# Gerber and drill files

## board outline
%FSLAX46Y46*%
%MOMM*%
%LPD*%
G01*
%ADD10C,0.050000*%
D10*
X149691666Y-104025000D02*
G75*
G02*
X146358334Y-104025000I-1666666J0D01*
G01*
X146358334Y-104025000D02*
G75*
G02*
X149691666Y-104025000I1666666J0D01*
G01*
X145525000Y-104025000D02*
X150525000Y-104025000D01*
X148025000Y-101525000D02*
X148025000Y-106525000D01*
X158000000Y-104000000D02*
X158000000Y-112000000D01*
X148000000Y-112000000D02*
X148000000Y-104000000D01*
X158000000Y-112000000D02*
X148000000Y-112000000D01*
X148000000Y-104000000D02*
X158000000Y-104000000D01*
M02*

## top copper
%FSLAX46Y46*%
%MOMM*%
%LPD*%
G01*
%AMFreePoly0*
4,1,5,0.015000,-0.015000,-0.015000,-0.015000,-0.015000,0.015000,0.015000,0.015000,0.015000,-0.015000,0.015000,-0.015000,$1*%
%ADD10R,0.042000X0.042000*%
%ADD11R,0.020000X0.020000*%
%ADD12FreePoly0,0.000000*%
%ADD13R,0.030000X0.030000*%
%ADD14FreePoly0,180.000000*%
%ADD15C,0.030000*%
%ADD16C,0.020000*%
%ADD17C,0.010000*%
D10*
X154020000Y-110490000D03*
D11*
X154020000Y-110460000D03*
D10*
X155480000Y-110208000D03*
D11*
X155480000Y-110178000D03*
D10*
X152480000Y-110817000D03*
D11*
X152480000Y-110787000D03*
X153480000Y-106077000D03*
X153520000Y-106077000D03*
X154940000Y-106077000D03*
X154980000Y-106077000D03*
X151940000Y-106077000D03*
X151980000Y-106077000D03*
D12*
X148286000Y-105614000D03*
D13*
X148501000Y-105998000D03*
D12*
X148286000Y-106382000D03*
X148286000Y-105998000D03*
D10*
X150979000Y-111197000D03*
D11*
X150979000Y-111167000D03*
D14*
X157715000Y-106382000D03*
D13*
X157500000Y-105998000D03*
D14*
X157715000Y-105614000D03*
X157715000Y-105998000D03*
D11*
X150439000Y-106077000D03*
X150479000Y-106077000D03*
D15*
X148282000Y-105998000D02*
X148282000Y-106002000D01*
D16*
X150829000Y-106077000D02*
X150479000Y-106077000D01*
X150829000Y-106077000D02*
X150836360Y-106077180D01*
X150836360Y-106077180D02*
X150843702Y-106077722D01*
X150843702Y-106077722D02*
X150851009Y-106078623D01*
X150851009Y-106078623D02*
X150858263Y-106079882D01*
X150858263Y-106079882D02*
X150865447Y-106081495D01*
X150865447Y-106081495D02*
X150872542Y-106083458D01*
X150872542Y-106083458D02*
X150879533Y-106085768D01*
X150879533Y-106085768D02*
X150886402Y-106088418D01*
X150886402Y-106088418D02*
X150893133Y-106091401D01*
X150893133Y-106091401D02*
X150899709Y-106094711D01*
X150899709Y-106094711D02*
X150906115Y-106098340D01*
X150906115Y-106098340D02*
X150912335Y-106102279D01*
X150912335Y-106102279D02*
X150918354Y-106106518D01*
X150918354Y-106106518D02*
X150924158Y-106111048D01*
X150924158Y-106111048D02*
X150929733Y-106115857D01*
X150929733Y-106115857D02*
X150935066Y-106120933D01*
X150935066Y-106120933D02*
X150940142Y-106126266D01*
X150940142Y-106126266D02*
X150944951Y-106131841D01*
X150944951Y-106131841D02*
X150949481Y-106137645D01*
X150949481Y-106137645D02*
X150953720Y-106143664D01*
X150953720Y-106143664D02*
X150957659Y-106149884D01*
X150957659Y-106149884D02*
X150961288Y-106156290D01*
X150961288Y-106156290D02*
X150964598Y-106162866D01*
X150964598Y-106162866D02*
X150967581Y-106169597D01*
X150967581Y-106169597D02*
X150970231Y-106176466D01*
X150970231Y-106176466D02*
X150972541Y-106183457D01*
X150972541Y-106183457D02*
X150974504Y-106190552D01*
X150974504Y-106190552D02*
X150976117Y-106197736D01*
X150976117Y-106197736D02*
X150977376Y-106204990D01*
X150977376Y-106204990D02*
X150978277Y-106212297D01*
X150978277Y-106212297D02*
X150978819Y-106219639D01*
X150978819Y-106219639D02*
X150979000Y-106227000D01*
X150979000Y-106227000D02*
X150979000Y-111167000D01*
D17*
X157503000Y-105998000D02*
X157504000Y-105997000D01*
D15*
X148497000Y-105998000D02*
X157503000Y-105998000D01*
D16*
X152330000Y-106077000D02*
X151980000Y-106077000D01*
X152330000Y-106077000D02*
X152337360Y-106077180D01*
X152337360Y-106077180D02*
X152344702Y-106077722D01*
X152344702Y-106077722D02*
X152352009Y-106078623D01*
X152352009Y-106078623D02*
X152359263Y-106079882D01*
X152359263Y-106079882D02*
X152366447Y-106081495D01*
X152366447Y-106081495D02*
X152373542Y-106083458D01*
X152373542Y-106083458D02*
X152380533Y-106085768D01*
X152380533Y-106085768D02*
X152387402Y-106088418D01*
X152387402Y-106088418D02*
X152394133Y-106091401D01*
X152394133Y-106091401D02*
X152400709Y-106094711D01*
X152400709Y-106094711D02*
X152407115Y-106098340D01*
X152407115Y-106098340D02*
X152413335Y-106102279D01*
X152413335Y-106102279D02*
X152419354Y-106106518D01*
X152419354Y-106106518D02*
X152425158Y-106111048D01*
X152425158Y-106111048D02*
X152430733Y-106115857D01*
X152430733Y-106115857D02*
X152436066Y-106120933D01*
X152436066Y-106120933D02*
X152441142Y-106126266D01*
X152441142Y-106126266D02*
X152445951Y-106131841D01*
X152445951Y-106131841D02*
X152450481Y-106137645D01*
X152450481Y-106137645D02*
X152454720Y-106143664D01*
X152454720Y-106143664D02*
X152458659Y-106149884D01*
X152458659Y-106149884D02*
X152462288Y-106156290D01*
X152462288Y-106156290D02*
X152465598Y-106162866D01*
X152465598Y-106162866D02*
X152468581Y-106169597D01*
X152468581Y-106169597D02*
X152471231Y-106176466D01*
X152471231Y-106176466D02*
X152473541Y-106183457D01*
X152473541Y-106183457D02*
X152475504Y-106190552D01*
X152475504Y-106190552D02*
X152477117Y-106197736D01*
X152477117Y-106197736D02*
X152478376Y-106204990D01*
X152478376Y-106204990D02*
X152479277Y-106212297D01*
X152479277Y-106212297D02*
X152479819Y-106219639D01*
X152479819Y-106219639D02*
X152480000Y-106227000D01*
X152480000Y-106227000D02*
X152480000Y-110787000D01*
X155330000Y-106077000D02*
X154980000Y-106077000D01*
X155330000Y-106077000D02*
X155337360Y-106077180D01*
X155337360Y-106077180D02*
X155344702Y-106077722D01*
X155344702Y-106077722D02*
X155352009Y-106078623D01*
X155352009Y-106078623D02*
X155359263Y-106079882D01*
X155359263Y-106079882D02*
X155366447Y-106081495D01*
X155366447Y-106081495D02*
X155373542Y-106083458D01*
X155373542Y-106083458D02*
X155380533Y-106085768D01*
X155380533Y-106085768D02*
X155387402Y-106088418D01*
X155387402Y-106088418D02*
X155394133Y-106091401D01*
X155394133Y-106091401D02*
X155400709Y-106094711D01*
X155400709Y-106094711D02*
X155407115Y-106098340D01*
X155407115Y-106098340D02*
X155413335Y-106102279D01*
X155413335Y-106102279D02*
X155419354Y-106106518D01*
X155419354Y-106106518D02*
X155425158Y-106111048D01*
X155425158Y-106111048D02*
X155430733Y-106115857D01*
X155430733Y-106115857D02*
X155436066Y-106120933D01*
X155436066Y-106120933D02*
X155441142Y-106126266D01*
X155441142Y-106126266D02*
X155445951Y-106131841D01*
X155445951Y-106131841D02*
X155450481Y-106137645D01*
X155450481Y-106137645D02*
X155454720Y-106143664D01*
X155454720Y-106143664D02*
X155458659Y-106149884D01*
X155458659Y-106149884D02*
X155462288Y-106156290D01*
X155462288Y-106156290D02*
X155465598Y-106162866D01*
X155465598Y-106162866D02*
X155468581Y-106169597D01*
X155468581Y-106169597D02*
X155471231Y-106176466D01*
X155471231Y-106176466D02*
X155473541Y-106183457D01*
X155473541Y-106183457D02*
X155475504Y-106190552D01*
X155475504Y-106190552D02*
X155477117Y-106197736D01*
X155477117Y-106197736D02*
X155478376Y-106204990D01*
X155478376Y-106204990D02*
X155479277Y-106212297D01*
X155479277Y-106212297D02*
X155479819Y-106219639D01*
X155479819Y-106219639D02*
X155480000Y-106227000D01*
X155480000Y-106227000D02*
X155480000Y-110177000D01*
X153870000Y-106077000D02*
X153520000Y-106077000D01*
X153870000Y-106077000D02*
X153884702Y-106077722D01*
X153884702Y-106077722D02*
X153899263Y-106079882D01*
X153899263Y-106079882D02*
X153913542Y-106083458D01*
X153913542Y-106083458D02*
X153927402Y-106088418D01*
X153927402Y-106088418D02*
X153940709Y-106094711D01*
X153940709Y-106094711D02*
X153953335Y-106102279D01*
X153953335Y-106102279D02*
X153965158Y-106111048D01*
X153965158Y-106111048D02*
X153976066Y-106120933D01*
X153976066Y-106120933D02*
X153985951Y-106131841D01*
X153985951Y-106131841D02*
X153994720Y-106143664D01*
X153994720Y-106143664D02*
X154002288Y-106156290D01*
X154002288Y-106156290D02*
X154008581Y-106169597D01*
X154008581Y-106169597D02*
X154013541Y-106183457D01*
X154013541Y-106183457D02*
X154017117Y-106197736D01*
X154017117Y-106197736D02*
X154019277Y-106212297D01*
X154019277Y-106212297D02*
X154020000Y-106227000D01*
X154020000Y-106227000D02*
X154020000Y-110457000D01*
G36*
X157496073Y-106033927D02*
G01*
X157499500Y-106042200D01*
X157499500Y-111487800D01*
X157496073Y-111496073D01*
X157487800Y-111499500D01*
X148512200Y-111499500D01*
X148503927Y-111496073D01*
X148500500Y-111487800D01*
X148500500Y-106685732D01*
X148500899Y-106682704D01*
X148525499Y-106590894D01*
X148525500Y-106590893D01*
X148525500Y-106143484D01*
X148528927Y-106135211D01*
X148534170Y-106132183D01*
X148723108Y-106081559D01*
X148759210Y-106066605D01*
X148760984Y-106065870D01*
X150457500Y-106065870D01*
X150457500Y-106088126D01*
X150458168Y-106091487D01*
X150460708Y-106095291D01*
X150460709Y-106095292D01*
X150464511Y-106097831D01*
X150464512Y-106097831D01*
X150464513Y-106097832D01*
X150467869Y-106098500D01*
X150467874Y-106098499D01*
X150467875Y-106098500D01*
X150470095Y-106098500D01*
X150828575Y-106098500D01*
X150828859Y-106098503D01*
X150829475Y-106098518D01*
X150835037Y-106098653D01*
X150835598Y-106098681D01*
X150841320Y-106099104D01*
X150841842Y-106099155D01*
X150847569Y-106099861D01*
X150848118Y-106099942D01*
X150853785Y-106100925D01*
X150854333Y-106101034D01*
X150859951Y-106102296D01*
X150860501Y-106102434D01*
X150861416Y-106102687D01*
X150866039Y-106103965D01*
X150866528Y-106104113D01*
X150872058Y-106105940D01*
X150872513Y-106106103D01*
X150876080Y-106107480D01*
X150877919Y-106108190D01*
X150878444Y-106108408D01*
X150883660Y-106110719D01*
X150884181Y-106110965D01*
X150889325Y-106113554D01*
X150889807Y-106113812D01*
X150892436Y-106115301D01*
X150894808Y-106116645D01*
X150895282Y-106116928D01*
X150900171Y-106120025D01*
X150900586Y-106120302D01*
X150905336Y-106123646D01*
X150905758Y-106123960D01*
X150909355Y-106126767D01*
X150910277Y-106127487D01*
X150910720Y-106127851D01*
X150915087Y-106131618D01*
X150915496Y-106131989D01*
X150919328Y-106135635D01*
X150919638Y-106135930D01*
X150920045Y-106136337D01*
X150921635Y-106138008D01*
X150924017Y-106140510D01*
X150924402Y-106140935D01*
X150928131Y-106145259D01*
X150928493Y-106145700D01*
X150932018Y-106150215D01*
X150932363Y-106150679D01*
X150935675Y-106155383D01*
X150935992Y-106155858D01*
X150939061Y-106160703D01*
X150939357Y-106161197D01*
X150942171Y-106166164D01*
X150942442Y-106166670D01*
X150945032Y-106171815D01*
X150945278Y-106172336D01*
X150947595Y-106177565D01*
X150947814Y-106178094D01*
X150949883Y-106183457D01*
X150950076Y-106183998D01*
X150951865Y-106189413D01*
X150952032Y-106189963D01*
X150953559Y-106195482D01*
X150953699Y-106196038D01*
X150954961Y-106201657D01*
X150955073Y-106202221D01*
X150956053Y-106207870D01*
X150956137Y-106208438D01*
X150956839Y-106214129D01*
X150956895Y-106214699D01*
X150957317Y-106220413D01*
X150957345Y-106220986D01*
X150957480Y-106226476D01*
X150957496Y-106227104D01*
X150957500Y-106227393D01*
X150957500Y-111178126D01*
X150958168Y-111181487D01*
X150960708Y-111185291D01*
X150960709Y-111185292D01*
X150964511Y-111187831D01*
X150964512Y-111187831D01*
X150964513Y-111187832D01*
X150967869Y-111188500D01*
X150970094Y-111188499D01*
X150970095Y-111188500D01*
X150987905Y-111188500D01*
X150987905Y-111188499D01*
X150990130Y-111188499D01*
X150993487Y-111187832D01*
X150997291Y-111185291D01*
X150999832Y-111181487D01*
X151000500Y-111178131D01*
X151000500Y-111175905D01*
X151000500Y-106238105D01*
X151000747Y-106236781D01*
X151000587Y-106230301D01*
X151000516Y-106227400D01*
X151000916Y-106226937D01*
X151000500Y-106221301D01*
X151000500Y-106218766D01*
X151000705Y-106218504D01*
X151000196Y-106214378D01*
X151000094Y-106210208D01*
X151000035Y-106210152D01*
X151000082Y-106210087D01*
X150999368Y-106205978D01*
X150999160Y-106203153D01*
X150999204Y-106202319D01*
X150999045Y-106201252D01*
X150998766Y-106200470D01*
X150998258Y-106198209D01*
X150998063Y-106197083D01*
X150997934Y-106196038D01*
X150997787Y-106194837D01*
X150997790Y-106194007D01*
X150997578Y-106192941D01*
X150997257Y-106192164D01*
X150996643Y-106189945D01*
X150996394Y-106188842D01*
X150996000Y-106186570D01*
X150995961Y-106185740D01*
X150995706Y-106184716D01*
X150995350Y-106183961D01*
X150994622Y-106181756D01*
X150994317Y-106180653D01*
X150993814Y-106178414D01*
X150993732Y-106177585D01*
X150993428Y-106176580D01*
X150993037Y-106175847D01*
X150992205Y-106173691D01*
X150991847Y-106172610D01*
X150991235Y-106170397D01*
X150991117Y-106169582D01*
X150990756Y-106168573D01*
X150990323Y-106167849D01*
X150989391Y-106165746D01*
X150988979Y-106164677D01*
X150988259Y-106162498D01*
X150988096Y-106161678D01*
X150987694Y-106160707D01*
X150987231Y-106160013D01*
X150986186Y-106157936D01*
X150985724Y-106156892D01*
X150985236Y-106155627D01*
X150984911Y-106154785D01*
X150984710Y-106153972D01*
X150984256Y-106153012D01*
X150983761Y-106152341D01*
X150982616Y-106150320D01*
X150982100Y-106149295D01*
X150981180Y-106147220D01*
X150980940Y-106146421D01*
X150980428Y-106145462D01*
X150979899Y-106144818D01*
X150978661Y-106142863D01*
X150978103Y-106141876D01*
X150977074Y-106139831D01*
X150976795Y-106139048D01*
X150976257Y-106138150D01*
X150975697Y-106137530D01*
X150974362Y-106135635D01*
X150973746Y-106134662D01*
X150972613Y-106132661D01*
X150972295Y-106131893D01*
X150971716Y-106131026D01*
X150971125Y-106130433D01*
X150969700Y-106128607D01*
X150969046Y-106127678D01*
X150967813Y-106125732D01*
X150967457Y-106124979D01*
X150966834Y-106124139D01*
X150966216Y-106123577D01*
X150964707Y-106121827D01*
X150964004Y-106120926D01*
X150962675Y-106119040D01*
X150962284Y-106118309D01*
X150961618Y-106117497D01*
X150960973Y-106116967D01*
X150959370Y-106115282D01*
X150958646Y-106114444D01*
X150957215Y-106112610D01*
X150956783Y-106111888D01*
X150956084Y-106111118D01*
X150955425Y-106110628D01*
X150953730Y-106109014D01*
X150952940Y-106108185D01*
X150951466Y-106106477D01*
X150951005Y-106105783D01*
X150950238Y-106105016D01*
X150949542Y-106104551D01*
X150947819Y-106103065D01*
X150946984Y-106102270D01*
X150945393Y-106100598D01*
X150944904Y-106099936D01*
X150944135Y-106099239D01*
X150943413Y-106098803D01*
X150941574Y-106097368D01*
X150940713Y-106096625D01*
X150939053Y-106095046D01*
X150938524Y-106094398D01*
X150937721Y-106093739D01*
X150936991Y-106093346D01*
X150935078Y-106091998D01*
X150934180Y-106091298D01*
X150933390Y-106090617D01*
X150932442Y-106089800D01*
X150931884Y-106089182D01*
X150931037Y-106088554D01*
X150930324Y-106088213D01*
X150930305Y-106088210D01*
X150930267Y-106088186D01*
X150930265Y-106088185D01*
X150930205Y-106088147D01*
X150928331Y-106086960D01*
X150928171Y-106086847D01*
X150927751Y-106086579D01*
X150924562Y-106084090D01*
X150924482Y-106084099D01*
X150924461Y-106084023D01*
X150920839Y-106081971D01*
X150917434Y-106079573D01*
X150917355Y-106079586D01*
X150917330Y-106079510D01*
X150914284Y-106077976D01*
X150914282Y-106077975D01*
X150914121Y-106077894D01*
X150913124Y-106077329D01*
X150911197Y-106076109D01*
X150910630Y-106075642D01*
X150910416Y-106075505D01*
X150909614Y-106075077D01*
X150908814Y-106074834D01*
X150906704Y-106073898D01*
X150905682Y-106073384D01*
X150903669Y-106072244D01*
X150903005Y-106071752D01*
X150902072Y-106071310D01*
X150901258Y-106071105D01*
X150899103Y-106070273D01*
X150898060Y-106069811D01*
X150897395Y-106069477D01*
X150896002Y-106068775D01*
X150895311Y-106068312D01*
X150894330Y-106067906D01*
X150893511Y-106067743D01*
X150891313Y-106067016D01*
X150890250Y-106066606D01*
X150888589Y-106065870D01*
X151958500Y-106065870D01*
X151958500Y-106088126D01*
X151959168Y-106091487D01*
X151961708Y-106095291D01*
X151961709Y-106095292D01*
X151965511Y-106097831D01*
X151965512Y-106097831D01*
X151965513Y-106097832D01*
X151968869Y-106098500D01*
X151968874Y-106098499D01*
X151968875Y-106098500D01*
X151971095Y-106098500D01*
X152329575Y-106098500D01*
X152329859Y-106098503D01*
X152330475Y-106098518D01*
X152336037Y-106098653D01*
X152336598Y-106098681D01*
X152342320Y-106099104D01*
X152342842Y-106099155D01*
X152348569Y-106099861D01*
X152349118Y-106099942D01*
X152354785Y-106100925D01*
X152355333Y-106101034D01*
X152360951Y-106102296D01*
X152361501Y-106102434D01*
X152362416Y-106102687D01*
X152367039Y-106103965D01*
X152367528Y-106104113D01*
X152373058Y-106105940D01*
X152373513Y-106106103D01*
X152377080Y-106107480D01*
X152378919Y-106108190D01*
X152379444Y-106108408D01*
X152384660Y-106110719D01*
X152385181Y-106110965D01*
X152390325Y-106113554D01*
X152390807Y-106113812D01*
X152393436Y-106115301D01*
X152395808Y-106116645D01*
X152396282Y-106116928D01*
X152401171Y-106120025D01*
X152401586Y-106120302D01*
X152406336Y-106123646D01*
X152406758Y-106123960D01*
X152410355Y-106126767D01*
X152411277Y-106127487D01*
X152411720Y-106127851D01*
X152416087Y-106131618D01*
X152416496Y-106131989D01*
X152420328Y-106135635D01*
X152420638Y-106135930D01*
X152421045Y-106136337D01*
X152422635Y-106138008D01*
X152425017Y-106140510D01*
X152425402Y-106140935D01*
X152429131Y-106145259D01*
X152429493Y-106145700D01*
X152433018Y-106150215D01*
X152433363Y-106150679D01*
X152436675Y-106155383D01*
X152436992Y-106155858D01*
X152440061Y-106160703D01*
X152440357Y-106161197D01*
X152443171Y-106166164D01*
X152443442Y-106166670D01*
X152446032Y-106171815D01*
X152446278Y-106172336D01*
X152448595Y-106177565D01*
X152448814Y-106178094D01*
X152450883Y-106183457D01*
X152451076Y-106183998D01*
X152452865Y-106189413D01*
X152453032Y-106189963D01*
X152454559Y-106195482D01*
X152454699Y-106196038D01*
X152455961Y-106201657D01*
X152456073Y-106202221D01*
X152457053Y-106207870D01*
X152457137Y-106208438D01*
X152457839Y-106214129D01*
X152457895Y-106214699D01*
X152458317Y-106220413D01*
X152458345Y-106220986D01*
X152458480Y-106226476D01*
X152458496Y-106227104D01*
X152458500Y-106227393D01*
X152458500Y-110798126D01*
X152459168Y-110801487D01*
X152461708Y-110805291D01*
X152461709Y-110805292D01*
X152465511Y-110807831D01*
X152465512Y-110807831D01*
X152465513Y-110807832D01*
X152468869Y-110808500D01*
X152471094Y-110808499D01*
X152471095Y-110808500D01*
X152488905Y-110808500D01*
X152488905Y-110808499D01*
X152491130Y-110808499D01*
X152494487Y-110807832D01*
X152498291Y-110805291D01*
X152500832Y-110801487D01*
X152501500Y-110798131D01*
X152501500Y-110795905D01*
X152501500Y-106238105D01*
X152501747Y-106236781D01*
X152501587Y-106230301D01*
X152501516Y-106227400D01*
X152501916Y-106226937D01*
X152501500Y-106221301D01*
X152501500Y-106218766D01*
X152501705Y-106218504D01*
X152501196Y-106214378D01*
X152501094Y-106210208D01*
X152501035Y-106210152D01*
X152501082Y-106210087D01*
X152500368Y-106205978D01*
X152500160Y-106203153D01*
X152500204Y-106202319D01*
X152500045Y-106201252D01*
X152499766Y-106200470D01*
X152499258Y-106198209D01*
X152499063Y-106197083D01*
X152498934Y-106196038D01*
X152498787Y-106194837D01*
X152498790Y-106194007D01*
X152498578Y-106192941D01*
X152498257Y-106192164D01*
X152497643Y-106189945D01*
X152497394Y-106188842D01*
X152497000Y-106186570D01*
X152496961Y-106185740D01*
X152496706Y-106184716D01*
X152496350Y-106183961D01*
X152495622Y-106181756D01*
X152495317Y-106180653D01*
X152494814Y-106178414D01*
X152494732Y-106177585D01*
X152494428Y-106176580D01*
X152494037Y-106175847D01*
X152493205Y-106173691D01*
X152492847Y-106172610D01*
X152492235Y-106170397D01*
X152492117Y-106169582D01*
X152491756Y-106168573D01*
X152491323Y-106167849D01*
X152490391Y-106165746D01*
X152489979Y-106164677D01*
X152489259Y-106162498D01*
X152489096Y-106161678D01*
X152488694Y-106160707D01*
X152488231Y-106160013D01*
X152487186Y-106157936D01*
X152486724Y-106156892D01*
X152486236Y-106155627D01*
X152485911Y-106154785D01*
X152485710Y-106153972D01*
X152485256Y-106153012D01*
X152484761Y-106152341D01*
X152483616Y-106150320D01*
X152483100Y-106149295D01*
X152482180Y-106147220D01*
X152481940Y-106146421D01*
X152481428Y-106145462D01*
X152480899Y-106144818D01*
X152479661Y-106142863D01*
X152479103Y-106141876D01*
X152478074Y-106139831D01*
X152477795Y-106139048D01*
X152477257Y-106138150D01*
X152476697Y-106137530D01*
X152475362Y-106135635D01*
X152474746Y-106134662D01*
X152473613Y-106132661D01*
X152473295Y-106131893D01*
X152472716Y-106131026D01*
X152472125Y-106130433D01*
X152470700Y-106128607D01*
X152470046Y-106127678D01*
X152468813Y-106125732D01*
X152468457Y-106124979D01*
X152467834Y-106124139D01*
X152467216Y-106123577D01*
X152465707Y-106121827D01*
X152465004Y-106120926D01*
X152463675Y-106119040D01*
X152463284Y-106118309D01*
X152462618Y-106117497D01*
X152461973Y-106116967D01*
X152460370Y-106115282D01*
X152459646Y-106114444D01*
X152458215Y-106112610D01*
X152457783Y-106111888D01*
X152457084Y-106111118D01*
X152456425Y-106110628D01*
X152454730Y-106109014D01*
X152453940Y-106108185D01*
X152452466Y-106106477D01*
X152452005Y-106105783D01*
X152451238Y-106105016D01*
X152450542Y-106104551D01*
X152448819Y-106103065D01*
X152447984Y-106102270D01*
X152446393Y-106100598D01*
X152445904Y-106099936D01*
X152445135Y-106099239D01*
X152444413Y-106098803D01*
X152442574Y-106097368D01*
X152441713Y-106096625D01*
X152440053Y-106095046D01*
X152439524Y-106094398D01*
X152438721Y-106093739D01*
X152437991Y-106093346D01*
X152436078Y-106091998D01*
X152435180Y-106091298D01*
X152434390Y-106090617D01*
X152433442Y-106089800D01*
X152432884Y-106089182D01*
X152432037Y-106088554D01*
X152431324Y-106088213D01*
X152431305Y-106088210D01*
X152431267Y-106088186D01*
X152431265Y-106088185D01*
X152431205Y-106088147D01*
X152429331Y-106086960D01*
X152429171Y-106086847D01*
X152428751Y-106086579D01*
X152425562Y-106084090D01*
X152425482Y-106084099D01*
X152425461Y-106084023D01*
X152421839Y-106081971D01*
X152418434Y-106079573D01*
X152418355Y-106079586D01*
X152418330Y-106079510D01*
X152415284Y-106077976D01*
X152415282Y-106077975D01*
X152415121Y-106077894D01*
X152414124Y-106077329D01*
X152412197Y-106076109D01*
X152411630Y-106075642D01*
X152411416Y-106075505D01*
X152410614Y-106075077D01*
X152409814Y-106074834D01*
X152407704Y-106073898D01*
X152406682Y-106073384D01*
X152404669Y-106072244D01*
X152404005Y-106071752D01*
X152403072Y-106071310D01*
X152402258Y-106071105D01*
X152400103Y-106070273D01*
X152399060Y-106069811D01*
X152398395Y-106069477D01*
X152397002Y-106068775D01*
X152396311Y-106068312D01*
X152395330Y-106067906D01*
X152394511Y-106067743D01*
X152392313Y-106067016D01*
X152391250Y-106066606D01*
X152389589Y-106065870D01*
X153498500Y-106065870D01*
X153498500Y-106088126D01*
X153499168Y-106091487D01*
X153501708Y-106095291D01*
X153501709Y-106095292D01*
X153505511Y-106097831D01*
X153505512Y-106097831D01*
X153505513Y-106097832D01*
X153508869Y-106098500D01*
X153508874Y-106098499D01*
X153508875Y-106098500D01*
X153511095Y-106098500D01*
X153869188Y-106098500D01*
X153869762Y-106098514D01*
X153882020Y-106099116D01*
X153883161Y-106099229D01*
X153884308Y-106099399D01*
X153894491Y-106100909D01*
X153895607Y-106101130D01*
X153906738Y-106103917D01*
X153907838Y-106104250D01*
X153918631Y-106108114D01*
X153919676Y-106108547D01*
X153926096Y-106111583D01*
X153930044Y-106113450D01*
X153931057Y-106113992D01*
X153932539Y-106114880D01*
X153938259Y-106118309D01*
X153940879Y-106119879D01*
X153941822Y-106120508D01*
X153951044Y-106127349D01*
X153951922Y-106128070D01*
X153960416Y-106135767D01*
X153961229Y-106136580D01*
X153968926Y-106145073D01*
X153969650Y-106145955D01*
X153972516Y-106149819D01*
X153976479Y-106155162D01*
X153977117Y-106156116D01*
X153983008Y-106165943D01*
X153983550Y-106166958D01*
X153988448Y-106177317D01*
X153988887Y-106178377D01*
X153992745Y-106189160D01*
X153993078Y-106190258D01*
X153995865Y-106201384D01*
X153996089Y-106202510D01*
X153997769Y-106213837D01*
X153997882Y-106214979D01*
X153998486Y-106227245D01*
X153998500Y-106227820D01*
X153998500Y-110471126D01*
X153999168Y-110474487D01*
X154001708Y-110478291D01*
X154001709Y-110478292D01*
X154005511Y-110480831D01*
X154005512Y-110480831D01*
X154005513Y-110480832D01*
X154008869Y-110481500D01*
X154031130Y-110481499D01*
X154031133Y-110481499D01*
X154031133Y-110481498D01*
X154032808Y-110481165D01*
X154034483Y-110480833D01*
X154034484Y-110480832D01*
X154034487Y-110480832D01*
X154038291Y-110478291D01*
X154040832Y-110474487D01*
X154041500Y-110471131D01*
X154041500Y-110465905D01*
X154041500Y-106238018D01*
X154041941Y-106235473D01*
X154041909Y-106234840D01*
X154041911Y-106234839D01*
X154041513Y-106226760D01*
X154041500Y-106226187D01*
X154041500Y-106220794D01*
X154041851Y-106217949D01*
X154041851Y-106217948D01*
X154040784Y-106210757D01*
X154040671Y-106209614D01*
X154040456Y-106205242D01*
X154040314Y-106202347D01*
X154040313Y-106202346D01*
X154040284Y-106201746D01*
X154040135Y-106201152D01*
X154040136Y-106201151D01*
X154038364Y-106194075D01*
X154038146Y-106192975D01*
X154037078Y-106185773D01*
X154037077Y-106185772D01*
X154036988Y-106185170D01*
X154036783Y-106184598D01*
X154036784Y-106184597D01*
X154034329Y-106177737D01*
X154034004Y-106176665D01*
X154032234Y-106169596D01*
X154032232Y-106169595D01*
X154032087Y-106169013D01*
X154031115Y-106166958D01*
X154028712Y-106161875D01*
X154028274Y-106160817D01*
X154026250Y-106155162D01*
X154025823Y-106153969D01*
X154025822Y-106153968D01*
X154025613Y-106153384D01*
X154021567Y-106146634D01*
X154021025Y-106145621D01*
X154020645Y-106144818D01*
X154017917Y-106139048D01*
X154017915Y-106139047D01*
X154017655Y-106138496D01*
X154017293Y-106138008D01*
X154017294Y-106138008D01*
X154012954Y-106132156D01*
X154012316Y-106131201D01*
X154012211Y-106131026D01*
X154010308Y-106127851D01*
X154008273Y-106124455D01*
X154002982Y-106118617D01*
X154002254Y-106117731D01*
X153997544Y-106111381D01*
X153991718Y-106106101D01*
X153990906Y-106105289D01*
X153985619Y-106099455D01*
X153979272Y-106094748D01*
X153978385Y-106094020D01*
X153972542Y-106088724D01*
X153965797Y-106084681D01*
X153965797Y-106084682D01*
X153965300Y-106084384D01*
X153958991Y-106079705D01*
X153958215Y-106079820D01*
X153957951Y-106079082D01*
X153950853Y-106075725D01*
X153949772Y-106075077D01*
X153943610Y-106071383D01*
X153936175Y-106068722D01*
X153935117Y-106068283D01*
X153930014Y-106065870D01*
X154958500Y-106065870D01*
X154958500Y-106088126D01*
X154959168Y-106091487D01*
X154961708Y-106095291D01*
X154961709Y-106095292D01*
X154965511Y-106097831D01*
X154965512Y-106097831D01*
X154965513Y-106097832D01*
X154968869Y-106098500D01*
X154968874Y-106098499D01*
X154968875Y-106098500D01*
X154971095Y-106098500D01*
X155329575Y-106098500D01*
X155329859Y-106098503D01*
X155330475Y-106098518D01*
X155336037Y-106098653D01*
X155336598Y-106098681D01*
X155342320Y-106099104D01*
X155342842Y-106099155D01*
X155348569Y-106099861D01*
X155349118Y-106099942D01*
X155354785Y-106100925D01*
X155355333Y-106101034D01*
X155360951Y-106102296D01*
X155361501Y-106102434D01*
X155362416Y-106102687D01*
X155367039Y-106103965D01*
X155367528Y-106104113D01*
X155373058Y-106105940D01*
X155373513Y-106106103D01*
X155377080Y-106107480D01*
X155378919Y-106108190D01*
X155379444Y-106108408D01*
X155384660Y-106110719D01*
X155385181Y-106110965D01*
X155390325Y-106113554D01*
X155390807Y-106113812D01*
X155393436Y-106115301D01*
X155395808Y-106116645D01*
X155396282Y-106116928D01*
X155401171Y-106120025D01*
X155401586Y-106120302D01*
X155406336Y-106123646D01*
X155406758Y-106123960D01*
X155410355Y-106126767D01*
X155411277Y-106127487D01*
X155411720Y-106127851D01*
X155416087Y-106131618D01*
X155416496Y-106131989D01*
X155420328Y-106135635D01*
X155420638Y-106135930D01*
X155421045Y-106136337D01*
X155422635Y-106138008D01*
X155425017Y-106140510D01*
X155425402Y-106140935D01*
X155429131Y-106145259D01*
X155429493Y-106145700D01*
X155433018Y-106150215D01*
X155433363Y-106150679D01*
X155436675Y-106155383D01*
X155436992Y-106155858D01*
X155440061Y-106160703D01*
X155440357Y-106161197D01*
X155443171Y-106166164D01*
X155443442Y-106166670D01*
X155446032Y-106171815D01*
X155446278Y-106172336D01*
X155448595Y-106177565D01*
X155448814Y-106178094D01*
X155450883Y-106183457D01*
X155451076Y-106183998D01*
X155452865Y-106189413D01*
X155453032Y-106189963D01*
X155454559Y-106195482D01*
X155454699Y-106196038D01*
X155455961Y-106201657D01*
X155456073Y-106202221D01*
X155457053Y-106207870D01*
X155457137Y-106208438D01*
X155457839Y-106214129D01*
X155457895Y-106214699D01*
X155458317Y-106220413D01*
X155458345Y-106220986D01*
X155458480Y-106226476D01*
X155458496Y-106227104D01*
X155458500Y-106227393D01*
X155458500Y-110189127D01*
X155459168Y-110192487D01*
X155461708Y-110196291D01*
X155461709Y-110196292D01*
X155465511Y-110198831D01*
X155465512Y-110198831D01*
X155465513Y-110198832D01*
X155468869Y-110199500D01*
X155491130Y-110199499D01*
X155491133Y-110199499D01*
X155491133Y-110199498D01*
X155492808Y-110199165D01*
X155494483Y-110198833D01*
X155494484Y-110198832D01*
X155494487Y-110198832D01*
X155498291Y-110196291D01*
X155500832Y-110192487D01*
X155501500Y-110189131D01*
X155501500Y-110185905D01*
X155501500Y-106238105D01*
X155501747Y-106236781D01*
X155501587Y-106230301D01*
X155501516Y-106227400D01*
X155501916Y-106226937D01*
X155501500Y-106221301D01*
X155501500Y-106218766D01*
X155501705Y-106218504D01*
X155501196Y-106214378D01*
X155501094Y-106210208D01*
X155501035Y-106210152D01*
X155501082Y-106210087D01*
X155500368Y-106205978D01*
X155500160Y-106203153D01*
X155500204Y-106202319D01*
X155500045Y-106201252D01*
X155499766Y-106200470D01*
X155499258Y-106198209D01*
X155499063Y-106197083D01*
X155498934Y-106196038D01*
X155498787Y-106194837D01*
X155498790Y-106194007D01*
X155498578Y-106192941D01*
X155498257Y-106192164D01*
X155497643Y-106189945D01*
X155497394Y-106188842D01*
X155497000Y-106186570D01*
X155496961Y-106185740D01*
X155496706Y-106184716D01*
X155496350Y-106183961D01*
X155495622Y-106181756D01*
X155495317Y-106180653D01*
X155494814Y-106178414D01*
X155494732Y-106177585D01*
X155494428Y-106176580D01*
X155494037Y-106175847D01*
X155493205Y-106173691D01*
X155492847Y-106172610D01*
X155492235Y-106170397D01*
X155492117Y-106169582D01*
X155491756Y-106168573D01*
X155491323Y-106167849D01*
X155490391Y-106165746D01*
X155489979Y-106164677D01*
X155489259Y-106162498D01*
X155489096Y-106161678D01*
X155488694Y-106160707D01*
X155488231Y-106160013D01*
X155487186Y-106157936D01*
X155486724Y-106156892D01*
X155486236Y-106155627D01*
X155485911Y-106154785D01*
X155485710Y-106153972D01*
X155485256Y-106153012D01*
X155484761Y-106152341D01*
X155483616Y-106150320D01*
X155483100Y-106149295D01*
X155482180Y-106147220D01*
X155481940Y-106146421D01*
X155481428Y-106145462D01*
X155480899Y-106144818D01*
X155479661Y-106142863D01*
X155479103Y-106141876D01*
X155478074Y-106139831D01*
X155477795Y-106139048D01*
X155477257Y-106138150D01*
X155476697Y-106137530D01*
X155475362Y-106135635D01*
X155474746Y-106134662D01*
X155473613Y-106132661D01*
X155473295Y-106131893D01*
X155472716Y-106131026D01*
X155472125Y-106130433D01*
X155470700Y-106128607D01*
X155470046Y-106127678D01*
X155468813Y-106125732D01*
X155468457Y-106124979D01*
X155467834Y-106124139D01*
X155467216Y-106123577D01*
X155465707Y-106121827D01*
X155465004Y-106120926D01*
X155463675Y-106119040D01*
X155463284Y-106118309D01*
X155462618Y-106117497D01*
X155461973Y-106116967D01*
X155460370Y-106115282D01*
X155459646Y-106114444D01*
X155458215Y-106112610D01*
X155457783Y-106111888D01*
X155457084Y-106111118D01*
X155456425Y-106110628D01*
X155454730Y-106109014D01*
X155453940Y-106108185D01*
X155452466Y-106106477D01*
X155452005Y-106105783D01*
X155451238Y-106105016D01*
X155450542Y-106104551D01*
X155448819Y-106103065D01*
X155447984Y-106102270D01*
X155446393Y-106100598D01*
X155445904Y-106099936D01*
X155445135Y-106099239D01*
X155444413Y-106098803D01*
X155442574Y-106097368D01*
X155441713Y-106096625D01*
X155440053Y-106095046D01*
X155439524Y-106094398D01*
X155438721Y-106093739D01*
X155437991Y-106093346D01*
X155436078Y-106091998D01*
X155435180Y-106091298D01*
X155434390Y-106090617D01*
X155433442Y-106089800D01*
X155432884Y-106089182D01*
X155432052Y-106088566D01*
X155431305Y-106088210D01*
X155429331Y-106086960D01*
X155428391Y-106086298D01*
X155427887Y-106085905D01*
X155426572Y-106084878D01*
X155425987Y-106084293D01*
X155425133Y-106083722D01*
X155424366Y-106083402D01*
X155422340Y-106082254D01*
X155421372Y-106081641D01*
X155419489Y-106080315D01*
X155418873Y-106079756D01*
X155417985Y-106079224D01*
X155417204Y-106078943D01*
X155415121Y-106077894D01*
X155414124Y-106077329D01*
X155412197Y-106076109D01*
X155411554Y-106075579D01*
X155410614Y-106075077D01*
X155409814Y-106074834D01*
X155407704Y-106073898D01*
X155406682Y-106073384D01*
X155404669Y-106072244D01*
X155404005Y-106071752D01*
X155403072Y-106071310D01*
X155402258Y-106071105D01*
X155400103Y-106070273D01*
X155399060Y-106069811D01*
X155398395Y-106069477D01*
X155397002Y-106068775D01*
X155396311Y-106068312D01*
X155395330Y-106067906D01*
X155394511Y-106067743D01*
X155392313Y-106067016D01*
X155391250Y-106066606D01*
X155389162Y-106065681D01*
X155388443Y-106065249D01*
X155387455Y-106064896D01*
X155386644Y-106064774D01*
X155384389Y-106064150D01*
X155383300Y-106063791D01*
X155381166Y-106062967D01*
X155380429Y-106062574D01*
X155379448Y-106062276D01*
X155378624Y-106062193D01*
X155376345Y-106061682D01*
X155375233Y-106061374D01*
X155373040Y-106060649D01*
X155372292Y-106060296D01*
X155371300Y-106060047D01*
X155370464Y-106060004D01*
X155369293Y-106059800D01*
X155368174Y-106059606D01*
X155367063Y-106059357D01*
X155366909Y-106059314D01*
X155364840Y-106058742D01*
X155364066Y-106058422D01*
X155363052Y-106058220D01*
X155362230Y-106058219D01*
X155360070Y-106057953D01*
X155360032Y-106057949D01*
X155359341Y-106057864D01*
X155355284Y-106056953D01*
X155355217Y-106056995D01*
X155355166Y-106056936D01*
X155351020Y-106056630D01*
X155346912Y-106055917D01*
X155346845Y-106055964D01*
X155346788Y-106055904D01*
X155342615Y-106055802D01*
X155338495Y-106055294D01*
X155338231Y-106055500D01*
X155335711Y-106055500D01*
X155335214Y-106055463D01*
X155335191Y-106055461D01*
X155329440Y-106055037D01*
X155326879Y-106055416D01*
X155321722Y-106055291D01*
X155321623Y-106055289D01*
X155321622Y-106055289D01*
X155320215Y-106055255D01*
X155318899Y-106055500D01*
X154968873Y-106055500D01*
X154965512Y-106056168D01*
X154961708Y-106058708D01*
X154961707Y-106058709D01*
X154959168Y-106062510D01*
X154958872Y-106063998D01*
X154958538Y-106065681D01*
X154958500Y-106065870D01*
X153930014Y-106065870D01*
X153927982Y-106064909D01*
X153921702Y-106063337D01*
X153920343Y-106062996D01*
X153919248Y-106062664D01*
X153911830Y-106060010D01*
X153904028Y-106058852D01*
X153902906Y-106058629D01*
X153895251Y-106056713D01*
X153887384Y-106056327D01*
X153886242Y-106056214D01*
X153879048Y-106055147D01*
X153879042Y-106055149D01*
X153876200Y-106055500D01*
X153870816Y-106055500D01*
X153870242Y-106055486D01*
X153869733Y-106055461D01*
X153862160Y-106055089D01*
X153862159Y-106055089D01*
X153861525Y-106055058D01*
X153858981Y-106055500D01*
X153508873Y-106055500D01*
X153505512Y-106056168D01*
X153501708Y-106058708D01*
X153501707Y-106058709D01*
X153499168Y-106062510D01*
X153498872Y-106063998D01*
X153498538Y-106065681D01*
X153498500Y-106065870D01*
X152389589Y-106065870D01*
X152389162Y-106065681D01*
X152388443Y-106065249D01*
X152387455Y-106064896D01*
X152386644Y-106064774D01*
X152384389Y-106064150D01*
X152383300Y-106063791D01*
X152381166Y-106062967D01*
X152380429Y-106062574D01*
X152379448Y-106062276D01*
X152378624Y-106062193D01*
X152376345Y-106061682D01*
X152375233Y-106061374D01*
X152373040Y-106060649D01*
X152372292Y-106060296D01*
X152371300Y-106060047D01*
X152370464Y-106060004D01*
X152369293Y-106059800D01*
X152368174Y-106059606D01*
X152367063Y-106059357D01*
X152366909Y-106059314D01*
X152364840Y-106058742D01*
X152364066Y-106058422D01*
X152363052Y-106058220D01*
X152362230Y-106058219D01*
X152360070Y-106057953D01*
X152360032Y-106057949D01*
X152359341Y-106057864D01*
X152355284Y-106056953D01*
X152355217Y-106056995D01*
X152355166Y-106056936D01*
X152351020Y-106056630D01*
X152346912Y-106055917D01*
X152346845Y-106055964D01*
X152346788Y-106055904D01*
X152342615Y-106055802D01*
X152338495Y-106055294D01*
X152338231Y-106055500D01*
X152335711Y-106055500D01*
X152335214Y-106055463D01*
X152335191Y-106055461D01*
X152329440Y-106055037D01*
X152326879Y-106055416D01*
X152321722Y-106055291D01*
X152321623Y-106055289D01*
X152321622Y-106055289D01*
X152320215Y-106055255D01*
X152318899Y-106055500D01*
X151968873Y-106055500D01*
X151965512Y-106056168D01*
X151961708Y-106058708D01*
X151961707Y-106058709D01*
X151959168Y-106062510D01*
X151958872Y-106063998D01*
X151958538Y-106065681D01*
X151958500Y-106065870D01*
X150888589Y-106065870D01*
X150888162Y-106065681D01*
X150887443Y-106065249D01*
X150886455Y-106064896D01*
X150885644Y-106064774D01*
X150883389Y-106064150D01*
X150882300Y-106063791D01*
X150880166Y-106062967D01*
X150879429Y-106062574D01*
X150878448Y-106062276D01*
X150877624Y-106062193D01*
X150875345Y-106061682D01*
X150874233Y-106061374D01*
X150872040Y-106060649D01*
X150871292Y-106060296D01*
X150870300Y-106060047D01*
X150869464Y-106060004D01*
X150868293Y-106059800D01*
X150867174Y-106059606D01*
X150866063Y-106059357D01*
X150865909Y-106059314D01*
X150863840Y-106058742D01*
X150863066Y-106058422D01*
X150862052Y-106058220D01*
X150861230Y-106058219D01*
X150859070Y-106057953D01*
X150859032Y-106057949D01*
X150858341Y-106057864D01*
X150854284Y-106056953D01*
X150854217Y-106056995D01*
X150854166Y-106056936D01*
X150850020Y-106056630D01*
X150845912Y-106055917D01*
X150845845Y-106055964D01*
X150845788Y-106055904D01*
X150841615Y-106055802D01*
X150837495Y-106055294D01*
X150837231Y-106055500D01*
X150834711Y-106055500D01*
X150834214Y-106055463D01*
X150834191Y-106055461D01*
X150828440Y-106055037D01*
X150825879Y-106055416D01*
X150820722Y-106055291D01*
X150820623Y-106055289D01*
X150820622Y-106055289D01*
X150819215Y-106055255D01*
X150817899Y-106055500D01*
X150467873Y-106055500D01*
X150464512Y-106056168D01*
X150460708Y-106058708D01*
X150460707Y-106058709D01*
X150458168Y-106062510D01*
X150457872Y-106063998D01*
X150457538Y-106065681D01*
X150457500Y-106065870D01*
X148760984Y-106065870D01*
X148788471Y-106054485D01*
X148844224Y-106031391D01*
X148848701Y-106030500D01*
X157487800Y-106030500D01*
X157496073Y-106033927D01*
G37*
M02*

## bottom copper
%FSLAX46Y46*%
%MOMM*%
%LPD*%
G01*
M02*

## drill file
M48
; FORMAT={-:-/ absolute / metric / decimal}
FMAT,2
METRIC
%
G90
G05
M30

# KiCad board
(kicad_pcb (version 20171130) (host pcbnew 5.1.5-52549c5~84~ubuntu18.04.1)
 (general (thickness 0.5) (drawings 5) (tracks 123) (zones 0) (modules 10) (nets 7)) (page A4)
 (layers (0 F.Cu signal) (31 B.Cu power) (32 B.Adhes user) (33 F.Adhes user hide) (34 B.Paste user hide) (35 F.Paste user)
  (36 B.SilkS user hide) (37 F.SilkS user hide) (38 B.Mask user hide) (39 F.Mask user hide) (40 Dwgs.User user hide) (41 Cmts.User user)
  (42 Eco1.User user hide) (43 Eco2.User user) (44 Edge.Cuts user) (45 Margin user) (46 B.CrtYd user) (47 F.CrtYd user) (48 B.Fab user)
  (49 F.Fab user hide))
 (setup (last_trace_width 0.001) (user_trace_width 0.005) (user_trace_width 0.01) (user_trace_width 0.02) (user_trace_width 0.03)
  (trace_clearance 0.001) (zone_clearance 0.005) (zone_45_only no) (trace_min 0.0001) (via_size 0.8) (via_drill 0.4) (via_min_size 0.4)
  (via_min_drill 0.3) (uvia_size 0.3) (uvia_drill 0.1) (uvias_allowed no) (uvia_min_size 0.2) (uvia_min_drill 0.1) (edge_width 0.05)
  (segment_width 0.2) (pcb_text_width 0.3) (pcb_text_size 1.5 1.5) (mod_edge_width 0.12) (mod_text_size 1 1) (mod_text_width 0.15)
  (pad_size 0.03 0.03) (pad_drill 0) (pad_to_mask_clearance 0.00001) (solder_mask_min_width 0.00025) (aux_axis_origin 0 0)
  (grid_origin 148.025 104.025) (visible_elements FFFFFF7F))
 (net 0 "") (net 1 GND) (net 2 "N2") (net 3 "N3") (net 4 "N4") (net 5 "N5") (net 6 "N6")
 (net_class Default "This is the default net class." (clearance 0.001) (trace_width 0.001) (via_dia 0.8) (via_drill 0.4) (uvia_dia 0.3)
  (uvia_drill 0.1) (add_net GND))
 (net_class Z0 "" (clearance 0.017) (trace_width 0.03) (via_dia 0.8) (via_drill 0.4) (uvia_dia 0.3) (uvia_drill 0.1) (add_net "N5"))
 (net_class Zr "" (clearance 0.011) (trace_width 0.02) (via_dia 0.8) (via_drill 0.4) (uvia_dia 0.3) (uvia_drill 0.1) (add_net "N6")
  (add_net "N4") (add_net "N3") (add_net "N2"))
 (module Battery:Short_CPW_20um (layer F.Cu) (at 154.02 110.46)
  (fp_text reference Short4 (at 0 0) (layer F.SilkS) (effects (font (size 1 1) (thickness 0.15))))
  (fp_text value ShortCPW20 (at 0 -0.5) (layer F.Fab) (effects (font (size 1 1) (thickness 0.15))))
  (pad 2 smd rect (at 0 0.03) (size 0.042 0.042) (layers F.Cu F.Paste F.Mask) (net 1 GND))
  (pad 1 smd rect (at 0 0) (size 0.02 0.02) (layers F.Cu F.Paste F.Mask) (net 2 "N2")))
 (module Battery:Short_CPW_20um (layer F.Cu) (at 155.48 110.178)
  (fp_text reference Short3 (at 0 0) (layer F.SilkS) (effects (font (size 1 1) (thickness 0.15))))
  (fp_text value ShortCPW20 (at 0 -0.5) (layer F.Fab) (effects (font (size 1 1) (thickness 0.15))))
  (pad 2 smd rect (at 0 0.03) (size 0.042 0.042) (layers F.Cu F.Paste F.Mask) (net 1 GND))
  (pad 1 smd rect (at 0 0) (size 0.02 0.02) (layers F.Cu F.Paste F.Mask) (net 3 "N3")))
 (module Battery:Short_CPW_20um (layer F.Cu) (at 152.48 110.787)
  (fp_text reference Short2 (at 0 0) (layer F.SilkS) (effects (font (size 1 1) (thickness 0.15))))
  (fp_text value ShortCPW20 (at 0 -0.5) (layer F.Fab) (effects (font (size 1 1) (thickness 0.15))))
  (pad 2 smd rect (at 0 0.03) (size 0.042 0.042) (layers F.Cu F.Paste F.Mask) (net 1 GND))
  (pad 1 smd rect (at 0 0) (size 0.02 0.02) (layers F.Cu F.Paste F.Mask) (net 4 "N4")))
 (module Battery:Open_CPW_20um (layer F.Cu) (at 153.52 106.077 270)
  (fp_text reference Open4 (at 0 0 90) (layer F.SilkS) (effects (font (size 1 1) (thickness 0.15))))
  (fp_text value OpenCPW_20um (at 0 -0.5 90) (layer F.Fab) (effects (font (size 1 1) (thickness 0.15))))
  (pad 2 smd rect (at 0 0.04 270) (size 0.02 0.02) (layers F.Cu F.Paste F.Mask) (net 1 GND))
  (pad 1 smd rect (at 0 0 270) (size 0.02 0.02) (layers F.Cu F.Paste F.Mask) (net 2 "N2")))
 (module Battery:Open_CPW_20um (layer F.Cu) (at 154.98 106.077 270)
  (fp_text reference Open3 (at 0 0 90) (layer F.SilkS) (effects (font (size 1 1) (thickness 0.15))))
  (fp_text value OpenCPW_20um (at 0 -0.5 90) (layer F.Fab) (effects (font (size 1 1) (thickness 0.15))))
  (pad 2 smd rect (at 0 0.04 270) (size 0.02 0.02) (layers F.Cu F.Paste F.Mask) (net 1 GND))
  (pad 1 smd rect (at 0 0 270) (size 0.02 0.02) (layers F.Cu F.Paste F.Mask) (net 3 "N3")))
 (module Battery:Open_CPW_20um (layer F.Cu) (at 151.98 106.077 270) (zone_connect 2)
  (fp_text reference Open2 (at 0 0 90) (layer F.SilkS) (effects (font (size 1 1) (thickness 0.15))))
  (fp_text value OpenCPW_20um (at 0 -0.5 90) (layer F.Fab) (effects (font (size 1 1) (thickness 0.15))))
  (pad 2 smd rect (at 0 0.04 270) (size 0.02 0.02) (layers F.Cu F.Paste F.Mask) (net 1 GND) (zone_connect 2))
  (pad 1 smd rect (at 0 0 270) (size 0.02 0.02) (layers F.Cu F.Paste F.Mask) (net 4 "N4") (zone_connect 2)))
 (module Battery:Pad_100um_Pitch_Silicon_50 (layer F.Cu) (at 148.286 105.998) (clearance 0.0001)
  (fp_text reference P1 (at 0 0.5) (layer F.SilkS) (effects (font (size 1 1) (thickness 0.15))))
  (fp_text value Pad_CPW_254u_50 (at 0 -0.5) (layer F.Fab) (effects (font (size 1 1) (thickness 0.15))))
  (pad 3 smd custom (at 0 -0.384) (size 0.03 0.03) (layers F.Cu F.Paste F.Mask) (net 1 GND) (clearance 0.001) (zone_connect 2)
   (options (clearance outline) (anchor rect)) (primitives))
  (pad 2 smd rect (at 0.215 0) (size 0.03 0.03) (layers F.Cu) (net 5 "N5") (clearance 0.001) (zone_connect 0))
  (pad 4 smd custom (at 0 0.384) (size 0.03 0.03) (layers F.Cu F.Paste F.Mask) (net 1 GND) (zone_connect 2)
   (options (clearance outline) (anchor rect)) (primitives))
  (pad 1 smd custom (at 0 0) (size 0.03 0.03) (layers F.Cu) (zone_connect 0) (options (clearance outline) (anchor rect)) (primitives)))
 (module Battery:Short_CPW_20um (layer F.Cu) (at 150.979 111.167)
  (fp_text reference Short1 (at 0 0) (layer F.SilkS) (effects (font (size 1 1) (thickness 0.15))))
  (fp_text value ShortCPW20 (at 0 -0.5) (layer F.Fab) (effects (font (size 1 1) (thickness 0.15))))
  (pad 2 smd rect (at 0 0.03) (size 0.042 0.042) (layers F.Cu F.Paste F.Mask) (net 1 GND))
  (pad 1 smd rect (at 0 0) (size 0.02 0.02) (layers F.Cu F.Paste F.Mask) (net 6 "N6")))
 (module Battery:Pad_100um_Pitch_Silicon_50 (layer F.Cu) (at 157.715 105.998 180) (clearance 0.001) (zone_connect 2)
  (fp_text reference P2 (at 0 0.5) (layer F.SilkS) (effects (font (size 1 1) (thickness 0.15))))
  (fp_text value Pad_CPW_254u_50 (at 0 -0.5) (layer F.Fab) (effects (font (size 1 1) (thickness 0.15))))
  (pad 4 smd custom (at 0 -0.384 180) (size 0.03 0.03) (layers *.Mask F.Cu F.Paste) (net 1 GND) (zone_connect 2)
   (options (clearance outline) (anchor rect)) (primitives))
  (pad 2 smd rect (at 0.215 0 180) (size 0.03 0.03) (layers F.Cu F.Paste F.Mask) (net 5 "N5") (zone_connect 0))
  (pad 3 smd custom (at 0 0.384 180) (size 0.03 0.03) (layers F.Cu F.Paste F.Mask) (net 1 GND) (zone_connect 2)
   (options (clearance convexhull) (anchor rect)) (primitives))
  (pad 1 smd custom (at 0 0 180) (size 0.03 0.03) (layers F.Cu F.Paste F.Mask) (zone_connect 0) (options (clearance outline) (anchor rect))
   (primitives)))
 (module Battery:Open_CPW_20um (layer F.Cu) (at 150.479 106.077 270)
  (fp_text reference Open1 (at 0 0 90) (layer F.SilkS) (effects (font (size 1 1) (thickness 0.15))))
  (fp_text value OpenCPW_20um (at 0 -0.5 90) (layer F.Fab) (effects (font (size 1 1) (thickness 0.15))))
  (pad 2 smd rect (at 0 0.04 270) (size 0.02 0.02) (layers F.Cu F.Paste F.Mask) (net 1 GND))
  (pad 1 smd rect (at 0 0 270) (size 0.02 0.02) (layers F.Cu F.Paste F.Mask) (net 6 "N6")))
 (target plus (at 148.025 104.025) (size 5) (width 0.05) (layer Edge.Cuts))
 (gr_line (start 158 104) (end 158 112) (layer Edge.Cuts) (width 0.05))
 (gr_line (start 148 112) (end 148 104) (layer Edge.Cuts) (width 0.05))
 (gr_line (start 158 112) (end 148 112) (layer Edge.Cuts) (width 0.05))
 (gr_line (start 148 104) (end 158 104) (layer Edge.Cuts) (width 0.05))
 (segment (start 148.282 105.998) (end 148.282 106.002) (width 0.03) (layer F.Cu) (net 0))
 (segment (start 150.829 106.077) (end 150.479 106.077) (width 0.02) (layer F.Cu) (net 6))
 (segment (start 150.829 106.077) (end 150.83636 106.07718) (width 0.02) (layer F.Cu) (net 6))
 (segment (start 150.83636 106.07718) (end 150.843702 106.077722) (width 0.02) (layer F.Cu) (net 6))
 (segment (start 150.843702 106.077722) (end 150.851009 106.078623) (width 0.02) (layer F.Cu) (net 6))
 (segment (start 150.851009 106.078623) (end 150.858263 106.079882) (width 0.02) (layer F.Cu) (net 6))
 (segment (start 150.858263 106.079882) (end 150.865447 106.081495) (width 0.02) (layer F.Cu) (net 6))
 (segment (start 150.865447 106.081495) (end 150.872542 106.083458) (width 0.02) (layer F.Cu) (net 6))
 (segment (start 150.872542 106.083458) (end 150.879533 106.085768) (width 0.02) (layer F.Cu) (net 6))
 (segment (start 150.879533 106.085768) (end 150.886402 106.088418) (width 0.02) (layer F.Cu) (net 6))
 (segment (start 150.886402 106.088418) (end 150.893133 106.091401) (width 0.02) (layer F.Cu) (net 6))
 (segment (start 150.893133 106.091401) (end 150.899709 106.094711) (width 0.02) (layer F.Cu) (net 6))
 (segment (start 150.899709 106.094711) (end 150.906115 106.09834) (width 0.02) (layer F.Cu) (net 6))
 (segment (start 150.906115 106.09834) (end 150.912335 106.102279) (width 0.02) (layer F.Cu) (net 6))
 (segment (start 150.912335 106.102279) (end 150.918354 106.106518) (width 0.02) (layer F.Cu) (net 6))
 (segment (start 150.918354 106.106518) (end 150.924158 106.111048) (width 0.02) (layer F.Cu) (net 6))
 (segment (start 150.924158 106.111048) (end 150.929733 106.115857) (width 0.02) (layer F.Cu) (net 6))
 (segment (start 150.929733 106.115857) (end 150.935066 106.120933) (width 0.02) (layer F.Cu) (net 6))
 (segment (start 150.935066 106.120933) (end 150.940142 106.126266) (width 0.02) (layer F.Cu) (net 6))
 (segment (start 150.940142 106.126266) (end 150.944951 106.131841) (width 0.02) (layer F.Cu) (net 6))
 (segment (start 150.944951 106.131841) (end 150.949481 106.137645) (width 0.02) (layer F.Cu) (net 6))
 (segment (start 150.949481 106.137645) (end 150.95372 106.143664) (width 0.02) (layer F.Cu) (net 6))
 (segment (start 150.95372 106.143664) (end 150.957659 106.149884) (width 0.02) (layer F.Cu) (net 6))
 (segment (start 150.957659 106.149884) (end 150.961288 106.15629) (width 0.02) (layer F.Cu) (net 6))
 (segment (start 150.961288 106.15629) (end 150.964598 106.162866) (width 0.02) (layer F.Cu) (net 6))
 (segment (start 150.964598 106.162866) (end 150.967581 106.169597) (width 0.02) (layer F.Cu) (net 6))
 (segment (start 150.967581 106.169597) (end 150.970231 106.176466) (width 0.02) (layer F.Cu) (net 6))
 (segment (start 150.970231 106.176466) (end 150.972541 106.183457) (width 0.02) (layer F.Cu) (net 6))
 (segment (start 150.972541 106.183457) (end 150.974504 106.190552) (width 0.02) (layer F.Cu) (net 6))
 (segment (start 150.974504 106.190552) (end 150.976117 106.197736) (width 0.02) (layer F.Cu) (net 6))
 (segment (start 150.976117 106.197736) (end 150.977376 106.20499) (width 0.02) (layer F.Cu) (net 6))
 (segment (start 150.977376 106.20499) (end 150.978277 106.212297) (width 0.02) (layer F.Cu) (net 6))
 (segment (start 150.978277 106.212297) (end 150.978819 106.219639) (width 0.02) (layer F.Cu) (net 6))
 (segment (start 150.978819 106.219639) (end 150.979 106.227) (width 0.02) (layer F.Cu) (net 6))
 (segment (start 150.979 106.227) (end 150.979 111.167) (width 0.02) (layer F.Cu) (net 6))
 (segment (start 157.503 105.998) (end 157.504 105.997) (width 0.01) (layer F.Cu) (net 5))
 (segment (start 148.497 105.998) (end 157.503 105.998) (width 0.03) (layer F.Cu) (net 5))
 (segment (start 152.33 106.077) (end 151.98 106.077) (width 0.02) (layer F.Cu) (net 4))
 (segment (start 152.33 106.077) (end 152.33736 106.07718) (width 0.02) (layer F.Cu) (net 4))
 (segment (start 152.33736 106.07718) (end 152.344702 106.077722) (width 0.02) (layer F.Cu) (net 4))
 (segment (start 152.344702 106.077722) (end 152.352009 106.078623) (width 0.02) (layer F.Cu) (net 4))
 (segment (start 152.352009 106.078623) (end 152.359263 106.079882) (width 0.02) (layer F.Cu) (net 4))
 (segment (start 152.359263 106.079882) (end 152.366447 106.081495) (width 0.02) (layer F.Cu) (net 4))
 (segment (start 152.366447 106.081495) (end 152.373542 106.083458) (width 0.02) (layer F.Cu) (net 4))
 (segment (start 152.373542 106.083458) (end 152.380533 106.085768) (width 0.02) (layer F.Cu) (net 4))
 (segment (start 152.380533 106.085768) (end 152.387402 106.088418) (width 0.02) (layer F.Cu) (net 4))
 (segment (start 152.387402 106.088418) (end 152.394133 106.091401) (width 0.02) (layer F.Cu) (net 4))
 (segment (start 152.394133 106.091401) (end 152.400709 106.094711) (width 0.02) (layer F.Cu) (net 4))
 (segment (start 152.400709 106.094711) (end 152.407115 106.09834) (width 0.02) (layer F.Cu) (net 4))
 (segment (start 152.407115 106.09834) (end 152.413335 106.102279) (width 0.02) (layer F.Cu) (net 4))
 (segment (start 152.413335 106.102279) (end 152.419354 106.106518) (width 0.02) (layer F.Cu) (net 4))
 (segment (start 152.419354 106.106518) (end 152.425158 106.111048) (width 0.02) (layer F.Cu) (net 4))
 (segment (start 152.425158 106.111048) (end 152.430733 106.115857) (width 0.02) (layer F.Cu) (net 4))
 (segment (start 152.430733 106.115857) (end 152.436066 106.120933) (width 0.02) (layer F.Cu) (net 4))
 (segment (start 152.436066 106.120933) (end 152.441142 106.126266) (width 0.02) (layer F.Cu) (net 4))
 (segment (start 152.441142 106.126266) (end 152.445951 106.131841) (width 0.02) (layer F.Cu) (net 4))
 (segment (start 152.445951 106.131841) (end 152.450481 106.137645) (width 0.02) (layer F.Cu) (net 4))
 (segment (start 152.450481 106.137645) (end 152.45472 106.143664) (width 0.02) (layer F.Cu) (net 4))
 (segment (start 152.45472 106.143664) (end 152.458659 106.149884) (width 0.02) (layer F.Cu) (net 4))
 (segment (start 152.458659 106.149884) (end 152.462288 106.15629) (width 0.02) (layer F.Cu) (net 4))
 (segment (start 152.462288 106.15629) (end 152.465598 106.162866) (width 0.02) (layer F.Cu) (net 4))
 (segment (start 152.465598 106.162866) (end 152.468581 106.169597) (width 0.02) (layer F.Cu) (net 4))
 (segment (start 152.468581 106.169597) (end 152.471231 106.176466) (width 0.02) (layer F.Cu) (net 4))
 (segment (start 152.471231 106.176466) (end 152.473541 106.183457) (width 0.02) (layer F.Cu) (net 4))
 (segment (start 152.473541 106.183457) (end 152.475504 106.190552) (width 0.02) (layer F.Cu) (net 4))
 (segment (start 152.475504 106.190552) (end 152.477117 106.197736) (width 0.02) (layer F.Cu) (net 4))
 (segment (start 152.477117 106.197736) (end 152.478376 106.20499) (width 0.02) (layer F.Cu) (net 4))
 (segment (start 152.478376 106.20499) (end 152.479277 106.212297) (width 0.02) (layer F.Cu) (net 4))
 (segment (start 152.479277 106.212297) (end 152.479819 106.219639) (width 0.02) (layer F.Cu) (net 4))
 (segment (start 152.479819 106.219639) (end 152.48 106.227) (width 0.02) (layer F.Cu) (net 4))
 (segment (start 152.48 106.227) (end 152.48 110.787) (width 0.02) (layer F.Cu) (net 4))
 (segment (start 155.33 106.077) (end 154.98 106.077) (width 0.02) (layer F.Cu) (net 3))
 (segment (start 155.33 106.077) (end 155.33736 106.07718) (width 0.02) (layer F.Cu) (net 3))
 (segment (start 155.33736 106.07718) (end 155.344702 106.077722) (width 0.02) (layer F.Cu) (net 3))
 (segment (start 155.344702 106.077722) (end 155.352009 106.078623) (width 0.02) (layer F.Cu) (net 3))
 (segment (start 155.352009 106.078623) (end 155.359263 106.079882) (width 0.02) (layer F.Cu) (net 3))
 (segment (start 155.359263 106.079882) (end 155.366447 106.081495) (width 0.02) (layer F.Cu) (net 3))
 (segment (start 155.366447 106.081495) (end 155.373542 106.083458) (width 0.02) (layer F.Cu) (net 3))
 (segment (start 155.373542 106.083458) (end 155.380533 106.085768) (width 0.02) (layer F.Cu) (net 3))
 (segment (start 155.380533 106.085768) (end 155.387402 106.088418) (width 0.02) (layer F.Cu) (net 3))
 (segment (start 155.387402 106.088418) (end 155.394133 106.091401) (width 0.02) (layer F.Cu) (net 3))
 (segment (start 155.394133 106.091401) (end 155.400709 106.094711) (width 0.02) (layer F.Cu) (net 3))
 (segment (start 155.400709 106.094711) (end 155.407115 106.09834) (width 0.02) (layer F.Cu) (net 3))
 (segment (start 155.407115 106.09834) (end 155.413335 106.102279) (width 0.02) (layer F.Cu) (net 3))
 (segment (start 155.413335 106.102279) (end 155.419354 106.106518) (width 0.02) (layer F.Cu) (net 3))
 (segment (start 155.419354 106.106518) (end 155.425158 106.111048) (width 0.02) (layer F.Cu) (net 3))
 (segment (start 155.425158 106.111048) (end 155.430733 106.115857) (width 0.02) (layer F.Cu) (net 3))
 (segment (start 155.430733 106.115857) (end 155.436066 106.120933) (width 0.02) (layer F.Cu) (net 3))
 (segment (start 155.436066 106.120933) (end 155.441142 106.126266) (width 0.02) (layer F.Cu) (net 3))
 (segment (start 155.441142 106.126266) (end 155.445951 106.131841) (width 0.02) (layer F.Cu) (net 3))
 (segment (start 155.445951 106.131841) (end 155.450481 106.137645) (width 0.02) (layer F.Cu) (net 3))
 (segment (start 155.450481 106.137645) (end 155.45472 106.143664) (width 0.02) (layer F.Cu) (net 3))
 (segment (start 155.45472 106.143664) (end 155.458659 106.149884) (width 0.02) (layer F.Cu) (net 3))
 (segment (start 155.458659 106.149884) (end 155.462288 106.15629) (width 0.02) (layer F.Cu) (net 3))
 (segment (start 155.462288 106.15629) (end 155.465598 106.162866) (width 0.02) (layer F.Cu) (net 3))
 (segment (start 155.465598 106.162866) (end 155.468581 106.169597) (width 0.02) (layer F.Cu) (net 3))
 (segment (start 155.468581 106.169597) (end 155.471231 106.176466) (width 0.02) (layer F.Cu) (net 3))
 (segment (start 155.471231 106.176466) (end 155.473541 106.183457) (width 0.02) (layer F.Cu) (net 3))
 (segment (start 155.473541 106.183457) (end 155.475504 106.190552) (width 0.02) (layer F.Cu) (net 3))
 (segment (start 155.475504 106.190552) (end 155.477117 106.197736) (width 0.02) (layer F.Cu) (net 3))
 (segment (start 155.477117 106.197736) (end 155.478376 106.20499) (width 0.02) (layer F.Cu) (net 3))
 (segment (start 155.478376 106.20499) (end 155.479277 106.212297) (width 0.02) (layer F.Cu) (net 3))
 (segment (start 155.479277 106.212297) (end 155.479819 106.219639) (width 0.02) (layer F.Cu) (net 3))
 (segment (start 155.479819 106.219639) (end 155.48 106.227) (width 0.02) (layer F.Cu) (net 3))
 (segment (start 155.48 106.227) (end 155.48 110.177) (width 0.02) (layer F.Cu) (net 3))
 (segment (start 153.87 106.077) (end 153.52 106.077) (width 0.02) (layer F.Cu) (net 2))
 (segment (start 153.87 106.077) (end 153.884702 106.077722) (width 0.02) (layer F.Cu) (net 2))
 (segment (start 153.884702 106.077722) (end 153.899263 106.079882) (width 0.02) (layer F.Cu) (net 2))
 (segment (start 153.899263 106.079882) (end 153.913542 106.083458) (width 0.02) (layer F.Cu) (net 2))
 (segment (start 153.913542 106.083458) (end 153.927402 106.088418) (width 0.02) (layer F.Cu) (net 2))
 (segment (start 153.927402 106.088418) (end 153.940709 106.094711) (width 0.02) (layer F.Cu) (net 2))
 (segment (start 153.940709 106.094711) (end 153.953335 106.102279) (width 0.02) (layer F.Cu) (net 2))
 (segment (start 153.953335 106.102279) (end 153.965158 106.111048) (width 0.02) (layer F.Cu) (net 2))
 (segment (start 153.965158 106.111048) (end 153.976066 106.120933) (width 0.02) (layer F.Cu) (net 2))
 (segment (start 153.976066 106.120933) (end 153.985951 106.131841) (width 0.02) (layer F.Cu) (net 2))
 (segment (start 153.985951 106.131841) (end 153.99472 106.143664) (width 0.02) (layer F.Cu) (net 2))
 (segment (start 153.99472 106.143664) (end 154.002288 106.15629) (width 0.02) (layer F.Cu) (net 2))
 (segment (start 154.002288 106.15629) (end 154.008581 106.169597) (width 0.02) (layer F.Cu) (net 2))
 (segment (start 154.008581 106.169597) (end 154.013541 106.183457) (width 0.02) (layer F.Cu) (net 2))
 (segment (start 154.013541 106.183457) (end 154.017117 106.197736) (width 0.02) (layer F.Cu) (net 2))
 (segment (start 154.017117 106.197736) (end 154.019277 106.212297) (width 0.02) (layer F.Cu) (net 2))
 (segment (start 154.019277 106.212297) (end 154.02 106.227) (width 0.02) (layer F.Cu) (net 2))
 (segment (start 154.02 106.227) (end 154.02 110.457) (width 0.02) (layer F.Cu) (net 2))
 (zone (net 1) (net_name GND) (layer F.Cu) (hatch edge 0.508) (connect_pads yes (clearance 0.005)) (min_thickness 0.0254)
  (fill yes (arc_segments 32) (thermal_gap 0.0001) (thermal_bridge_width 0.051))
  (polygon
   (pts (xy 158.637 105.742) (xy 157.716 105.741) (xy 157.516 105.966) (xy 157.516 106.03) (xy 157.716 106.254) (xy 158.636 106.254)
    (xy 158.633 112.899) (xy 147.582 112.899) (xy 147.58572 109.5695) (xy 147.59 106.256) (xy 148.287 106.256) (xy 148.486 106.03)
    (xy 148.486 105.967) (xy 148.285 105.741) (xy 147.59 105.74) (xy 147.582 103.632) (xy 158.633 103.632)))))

